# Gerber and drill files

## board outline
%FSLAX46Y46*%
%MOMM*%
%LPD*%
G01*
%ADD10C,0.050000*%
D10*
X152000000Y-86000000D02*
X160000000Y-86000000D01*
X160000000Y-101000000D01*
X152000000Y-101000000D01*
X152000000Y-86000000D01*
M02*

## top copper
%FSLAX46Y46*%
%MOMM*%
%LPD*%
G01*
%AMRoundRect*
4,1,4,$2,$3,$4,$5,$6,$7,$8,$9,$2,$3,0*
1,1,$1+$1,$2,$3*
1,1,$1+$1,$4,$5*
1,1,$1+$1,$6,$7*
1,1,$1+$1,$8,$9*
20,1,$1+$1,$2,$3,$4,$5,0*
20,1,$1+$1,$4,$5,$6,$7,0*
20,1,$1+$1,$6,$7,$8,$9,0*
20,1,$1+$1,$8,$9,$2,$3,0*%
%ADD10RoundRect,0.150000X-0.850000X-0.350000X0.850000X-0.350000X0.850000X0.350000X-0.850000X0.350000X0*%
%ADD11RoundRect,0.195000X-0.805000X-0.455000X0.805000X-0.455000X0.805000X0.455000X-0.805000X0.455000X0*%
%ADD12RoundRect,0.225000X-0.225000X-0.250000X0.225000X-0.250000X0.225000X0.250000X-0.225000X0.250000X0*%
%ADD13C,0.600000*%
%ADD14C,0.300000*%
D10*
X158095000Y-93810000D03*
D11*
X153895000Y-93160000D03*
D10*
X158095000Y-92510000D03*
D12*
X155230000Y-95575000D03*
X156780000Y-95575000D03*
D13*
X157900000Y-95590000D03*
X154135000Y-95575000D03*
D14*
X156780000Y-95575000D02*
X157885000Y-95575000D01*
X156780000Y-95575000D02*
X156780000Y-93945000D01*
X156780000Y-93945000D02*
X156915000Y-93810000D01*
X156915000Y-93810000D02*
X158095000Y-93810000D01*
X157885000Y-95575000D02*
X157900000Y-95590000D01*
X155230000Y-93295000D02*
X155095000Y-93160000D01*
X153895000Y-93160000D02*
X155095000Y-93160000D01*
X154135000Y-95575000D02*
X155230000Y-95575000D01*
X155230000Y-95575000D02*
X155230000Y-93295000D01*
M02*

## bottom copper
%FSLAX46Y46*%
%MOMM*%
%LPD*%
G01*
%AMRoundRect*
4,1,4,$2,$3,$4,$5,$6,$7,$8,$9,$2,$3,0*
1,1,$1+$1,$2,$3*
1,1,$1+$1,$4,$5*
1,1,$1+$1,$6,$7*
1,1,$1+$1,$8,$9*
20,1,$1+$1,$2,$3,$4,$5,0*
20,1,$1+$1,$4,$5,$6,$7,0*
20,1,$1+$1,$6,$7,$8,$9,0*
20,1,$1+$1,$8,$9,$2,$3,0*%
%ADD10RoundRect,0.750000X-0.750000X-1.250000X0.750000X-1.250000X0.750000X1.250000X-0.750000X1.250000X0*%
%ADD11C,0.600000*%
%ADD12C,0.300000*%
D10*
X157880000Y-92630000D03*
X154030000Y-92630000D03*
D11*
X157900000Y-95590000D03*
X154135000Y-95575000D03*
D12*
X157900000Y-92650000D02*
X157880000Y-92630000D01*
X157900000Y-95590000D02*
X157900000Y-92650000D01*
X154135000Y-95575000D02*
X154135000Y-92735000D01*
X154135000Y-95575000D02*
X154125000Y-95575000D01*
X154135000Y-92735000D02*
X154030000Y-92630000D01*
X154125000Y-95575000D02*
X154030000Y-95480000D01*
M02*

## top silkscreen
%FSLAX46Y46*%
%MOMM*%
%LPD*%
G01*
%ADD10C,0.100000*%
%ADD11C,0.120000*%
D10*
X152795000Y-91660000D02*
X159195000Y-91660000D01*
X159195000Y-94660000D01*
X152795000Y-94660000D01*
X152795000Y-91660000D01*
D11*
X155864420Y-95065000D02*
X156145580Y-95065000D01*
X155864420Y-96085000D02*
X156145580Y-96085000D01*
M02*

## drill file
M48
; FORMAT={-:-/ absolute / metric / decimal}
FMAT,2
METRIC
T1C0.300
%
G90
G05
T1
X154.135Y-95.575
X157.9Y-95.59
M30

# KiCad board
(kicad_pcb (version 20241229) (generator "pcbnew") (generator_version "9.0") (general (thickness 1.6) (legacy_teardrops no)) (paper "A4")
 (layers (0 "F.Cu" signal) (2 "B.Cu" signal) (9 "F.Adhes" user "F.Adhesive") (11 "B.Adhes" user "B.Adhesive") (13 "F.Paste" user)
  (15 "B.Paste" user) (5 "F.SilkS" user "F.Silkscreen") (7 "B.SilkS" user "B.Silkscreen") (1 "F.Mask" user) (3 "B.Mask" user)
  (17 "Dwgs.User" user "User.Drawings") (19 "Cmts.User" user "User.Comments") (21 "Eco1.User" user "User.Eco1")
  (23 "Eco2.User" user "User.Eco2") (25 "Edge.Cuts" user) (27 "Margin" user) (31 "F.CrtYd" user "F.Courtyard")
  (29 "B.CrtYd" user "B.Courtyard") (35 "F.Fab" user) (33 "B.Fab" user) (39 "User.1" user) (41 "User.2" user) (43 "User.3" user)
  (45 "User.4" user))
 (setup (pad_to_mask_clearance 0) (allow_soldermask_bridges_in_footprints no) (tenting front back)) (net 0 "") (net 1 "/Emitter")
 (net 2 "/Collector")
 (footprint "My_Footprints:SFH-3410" (layer "F.Cu") (at 156.005 93.18)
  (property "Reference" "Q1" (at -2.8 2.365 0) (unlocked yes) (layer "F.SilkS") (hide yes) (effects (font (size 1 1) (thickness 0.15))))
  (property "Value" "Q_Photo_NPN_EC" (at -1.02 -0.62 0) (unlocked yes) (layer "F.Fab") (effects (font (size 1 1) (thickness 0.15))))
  (fp_rect (start -3.21 -1.52) (end 3.19 1.48) (stroke (width 0.1) (type solid)) (fill no) (layer "F.SilkS"))
  (pad "1" smd roundrect (at 2.09 0.63) (size 2 1) (layers "F.Cu" "F.Mask" "F.Paste") (roundrect_rratio 0.15) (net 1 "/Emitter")
   (thermal_bridge_angle 45))
  (pad "2" smd roundrect (at -2.11 -0.02) (size 2 1.3) (layers "F.Cu" "F.Mask" "F.Paste") (roundrect_rratio 0.15) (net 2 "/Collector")
   (thermal_bridge_angle 45))
  (pad "3" smd roundrect (at 2.09 -0.67) (size 2 1) (layers "F.Cu" "F.Mask" "F.Paste") (roundrect_rratio 0.15) (thermal_bridge_angle 45)))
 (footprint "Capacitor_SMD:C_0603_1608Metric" (layer "F.Cu") (at 156.005 95.575)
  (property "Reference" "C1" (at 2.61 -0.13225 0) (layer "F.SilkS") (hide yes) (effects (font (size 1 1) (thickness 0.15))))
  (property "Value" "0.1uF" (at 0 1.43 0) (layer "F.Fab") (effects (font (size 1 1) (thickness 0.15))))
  (fp_line (start -0.14058 -0.51) (end 0.14058 -0.51) (stroke (width 0.12) (type solid)) (layer "F.SilkS"))
  (fp_line (start -0.14058 0.51) (end 0.14058 0.51) (stroke (width 0.12) (type solid)) (layer "F.SilkS"))
  (pad "1" smd roundrect (at -0.775 0) (size 0.9 0.95) (layers "F.Cu" "F.Mask" "F.Paste") (roundrect_rratio 0.25) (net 2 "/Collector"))
  (pad "2" smd roundrect (at 0.775 0) (size 0.9 0.95) (layers "F.Cu" "F.Mask" "F.Paste") (roundrect_rratio 0.25) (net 1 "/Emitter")))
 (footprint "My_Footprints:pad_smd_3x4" (layer "B.Cu") (at 158.08 92.63 90)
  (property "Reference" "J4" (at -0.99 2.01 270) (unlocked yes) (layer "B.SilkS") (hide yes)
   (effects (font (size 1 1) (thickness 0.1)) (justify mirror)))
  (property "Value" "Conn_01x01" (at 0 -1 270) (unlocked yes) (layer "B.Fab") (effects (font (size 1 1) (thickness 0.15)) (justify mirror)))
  (pad "1" smd roundrect (at 0 -0.2) (size 3 4) (layers "B.Cu" "B.Mask" "B.Paste") (roundrect_rratio 0.25) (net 1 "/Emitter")
   (thermal_bridge_angle 45)))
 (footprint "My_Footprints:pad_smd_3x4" (layer "B.Cu") (at 154.23 92.63 90)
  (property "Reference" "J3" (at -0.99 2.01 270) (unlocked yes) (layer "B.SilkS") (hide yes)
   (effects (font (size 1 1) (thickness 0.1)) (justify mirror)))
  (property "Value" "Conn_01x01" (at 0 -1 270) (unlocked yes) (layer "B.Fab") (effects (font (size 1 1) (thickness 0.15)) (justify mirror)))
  (pad "1" smd roundrect (at 0 -0.2) (size 3 4) (layers "B.Cu" "B.Mask" "B.Paste") (roundrect_rratio 0.25) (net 2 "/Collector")
   (thermal_bridge_angle 45)))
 (gr_rect (start 152 86) (end 160 101) (stroke (width 0.05) (type solid)) (fill no) (layer "Edge.Cuts"))
 (segment (start 156.78 95.575) (end 157.885 95.575) (width 0.3) (layer "F.Cu") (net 1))
 (segment (start 156.78 95.575) (end 156.78 93.945) (width 0.3) (layer "F.Cu") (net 1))
 (segment (start 156.78 93.945) (end 156.915 93.81) (width 0.3) (layer "F.Cu") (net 1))
 (segment (start 156.915 93.81) (end 158.095 93.81) (width 0.3) (layer "F.Cu") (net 1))
 (segment (start 157.885 95.575) (end 157.9 95.59) (width 0.3) (layer "F.Cu") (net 1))
 (via (at 157.9 95.59) (size 0.6) (drill 0.3) (layers "F.Cu" "B.Cu") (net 1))
 (segment (start 157.9 92.65) (end 157.88 92.63) (width 0.3) (layer "B.Cu") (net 1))
 (segment (start 157.9 95.59) (end 157.9 92.65) (width 0.3) (layer "B.Cu") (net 1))
 (segment (start 155.23 93.295) (end 155.095 93.16) (width 0.3) (layer "F.Cu") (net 2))
 (segment (start 153.895 93.16) (end 155.095 93.16) (width 0.3) (layer "F.Cu") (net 2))
 (segment (start 154.135 95.575) (end 155.23 95.575) (width 0.3) (layer "F.Cu") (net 2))
 (segment (start 155.23 95.575) (end 155.23 93.295) (width 0.3) (layer "F.Cu") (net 2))
 (via (at 154.135 95.575) (size 0.6) (drill 0.3) (layers "F.Cu" "B.Cu") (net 2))
 (segment (start 154.135 95.575) (end 154.135 92.735) (width 0.3) (layer "B.Cu") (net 2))
 (segment (start 154.135 95.575) (end 154.125 95.575) (width 0.3) (layer "B.Cu") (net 2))
 (segment (start 154.135 92.735) (end 154.03 92.63) (width 0.3) (layer "B.Cu") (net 2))
 (segment (start 154.125 95.575) (end 154.03 95.48) (width 0.3) (layer "B.Cu") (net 2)))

